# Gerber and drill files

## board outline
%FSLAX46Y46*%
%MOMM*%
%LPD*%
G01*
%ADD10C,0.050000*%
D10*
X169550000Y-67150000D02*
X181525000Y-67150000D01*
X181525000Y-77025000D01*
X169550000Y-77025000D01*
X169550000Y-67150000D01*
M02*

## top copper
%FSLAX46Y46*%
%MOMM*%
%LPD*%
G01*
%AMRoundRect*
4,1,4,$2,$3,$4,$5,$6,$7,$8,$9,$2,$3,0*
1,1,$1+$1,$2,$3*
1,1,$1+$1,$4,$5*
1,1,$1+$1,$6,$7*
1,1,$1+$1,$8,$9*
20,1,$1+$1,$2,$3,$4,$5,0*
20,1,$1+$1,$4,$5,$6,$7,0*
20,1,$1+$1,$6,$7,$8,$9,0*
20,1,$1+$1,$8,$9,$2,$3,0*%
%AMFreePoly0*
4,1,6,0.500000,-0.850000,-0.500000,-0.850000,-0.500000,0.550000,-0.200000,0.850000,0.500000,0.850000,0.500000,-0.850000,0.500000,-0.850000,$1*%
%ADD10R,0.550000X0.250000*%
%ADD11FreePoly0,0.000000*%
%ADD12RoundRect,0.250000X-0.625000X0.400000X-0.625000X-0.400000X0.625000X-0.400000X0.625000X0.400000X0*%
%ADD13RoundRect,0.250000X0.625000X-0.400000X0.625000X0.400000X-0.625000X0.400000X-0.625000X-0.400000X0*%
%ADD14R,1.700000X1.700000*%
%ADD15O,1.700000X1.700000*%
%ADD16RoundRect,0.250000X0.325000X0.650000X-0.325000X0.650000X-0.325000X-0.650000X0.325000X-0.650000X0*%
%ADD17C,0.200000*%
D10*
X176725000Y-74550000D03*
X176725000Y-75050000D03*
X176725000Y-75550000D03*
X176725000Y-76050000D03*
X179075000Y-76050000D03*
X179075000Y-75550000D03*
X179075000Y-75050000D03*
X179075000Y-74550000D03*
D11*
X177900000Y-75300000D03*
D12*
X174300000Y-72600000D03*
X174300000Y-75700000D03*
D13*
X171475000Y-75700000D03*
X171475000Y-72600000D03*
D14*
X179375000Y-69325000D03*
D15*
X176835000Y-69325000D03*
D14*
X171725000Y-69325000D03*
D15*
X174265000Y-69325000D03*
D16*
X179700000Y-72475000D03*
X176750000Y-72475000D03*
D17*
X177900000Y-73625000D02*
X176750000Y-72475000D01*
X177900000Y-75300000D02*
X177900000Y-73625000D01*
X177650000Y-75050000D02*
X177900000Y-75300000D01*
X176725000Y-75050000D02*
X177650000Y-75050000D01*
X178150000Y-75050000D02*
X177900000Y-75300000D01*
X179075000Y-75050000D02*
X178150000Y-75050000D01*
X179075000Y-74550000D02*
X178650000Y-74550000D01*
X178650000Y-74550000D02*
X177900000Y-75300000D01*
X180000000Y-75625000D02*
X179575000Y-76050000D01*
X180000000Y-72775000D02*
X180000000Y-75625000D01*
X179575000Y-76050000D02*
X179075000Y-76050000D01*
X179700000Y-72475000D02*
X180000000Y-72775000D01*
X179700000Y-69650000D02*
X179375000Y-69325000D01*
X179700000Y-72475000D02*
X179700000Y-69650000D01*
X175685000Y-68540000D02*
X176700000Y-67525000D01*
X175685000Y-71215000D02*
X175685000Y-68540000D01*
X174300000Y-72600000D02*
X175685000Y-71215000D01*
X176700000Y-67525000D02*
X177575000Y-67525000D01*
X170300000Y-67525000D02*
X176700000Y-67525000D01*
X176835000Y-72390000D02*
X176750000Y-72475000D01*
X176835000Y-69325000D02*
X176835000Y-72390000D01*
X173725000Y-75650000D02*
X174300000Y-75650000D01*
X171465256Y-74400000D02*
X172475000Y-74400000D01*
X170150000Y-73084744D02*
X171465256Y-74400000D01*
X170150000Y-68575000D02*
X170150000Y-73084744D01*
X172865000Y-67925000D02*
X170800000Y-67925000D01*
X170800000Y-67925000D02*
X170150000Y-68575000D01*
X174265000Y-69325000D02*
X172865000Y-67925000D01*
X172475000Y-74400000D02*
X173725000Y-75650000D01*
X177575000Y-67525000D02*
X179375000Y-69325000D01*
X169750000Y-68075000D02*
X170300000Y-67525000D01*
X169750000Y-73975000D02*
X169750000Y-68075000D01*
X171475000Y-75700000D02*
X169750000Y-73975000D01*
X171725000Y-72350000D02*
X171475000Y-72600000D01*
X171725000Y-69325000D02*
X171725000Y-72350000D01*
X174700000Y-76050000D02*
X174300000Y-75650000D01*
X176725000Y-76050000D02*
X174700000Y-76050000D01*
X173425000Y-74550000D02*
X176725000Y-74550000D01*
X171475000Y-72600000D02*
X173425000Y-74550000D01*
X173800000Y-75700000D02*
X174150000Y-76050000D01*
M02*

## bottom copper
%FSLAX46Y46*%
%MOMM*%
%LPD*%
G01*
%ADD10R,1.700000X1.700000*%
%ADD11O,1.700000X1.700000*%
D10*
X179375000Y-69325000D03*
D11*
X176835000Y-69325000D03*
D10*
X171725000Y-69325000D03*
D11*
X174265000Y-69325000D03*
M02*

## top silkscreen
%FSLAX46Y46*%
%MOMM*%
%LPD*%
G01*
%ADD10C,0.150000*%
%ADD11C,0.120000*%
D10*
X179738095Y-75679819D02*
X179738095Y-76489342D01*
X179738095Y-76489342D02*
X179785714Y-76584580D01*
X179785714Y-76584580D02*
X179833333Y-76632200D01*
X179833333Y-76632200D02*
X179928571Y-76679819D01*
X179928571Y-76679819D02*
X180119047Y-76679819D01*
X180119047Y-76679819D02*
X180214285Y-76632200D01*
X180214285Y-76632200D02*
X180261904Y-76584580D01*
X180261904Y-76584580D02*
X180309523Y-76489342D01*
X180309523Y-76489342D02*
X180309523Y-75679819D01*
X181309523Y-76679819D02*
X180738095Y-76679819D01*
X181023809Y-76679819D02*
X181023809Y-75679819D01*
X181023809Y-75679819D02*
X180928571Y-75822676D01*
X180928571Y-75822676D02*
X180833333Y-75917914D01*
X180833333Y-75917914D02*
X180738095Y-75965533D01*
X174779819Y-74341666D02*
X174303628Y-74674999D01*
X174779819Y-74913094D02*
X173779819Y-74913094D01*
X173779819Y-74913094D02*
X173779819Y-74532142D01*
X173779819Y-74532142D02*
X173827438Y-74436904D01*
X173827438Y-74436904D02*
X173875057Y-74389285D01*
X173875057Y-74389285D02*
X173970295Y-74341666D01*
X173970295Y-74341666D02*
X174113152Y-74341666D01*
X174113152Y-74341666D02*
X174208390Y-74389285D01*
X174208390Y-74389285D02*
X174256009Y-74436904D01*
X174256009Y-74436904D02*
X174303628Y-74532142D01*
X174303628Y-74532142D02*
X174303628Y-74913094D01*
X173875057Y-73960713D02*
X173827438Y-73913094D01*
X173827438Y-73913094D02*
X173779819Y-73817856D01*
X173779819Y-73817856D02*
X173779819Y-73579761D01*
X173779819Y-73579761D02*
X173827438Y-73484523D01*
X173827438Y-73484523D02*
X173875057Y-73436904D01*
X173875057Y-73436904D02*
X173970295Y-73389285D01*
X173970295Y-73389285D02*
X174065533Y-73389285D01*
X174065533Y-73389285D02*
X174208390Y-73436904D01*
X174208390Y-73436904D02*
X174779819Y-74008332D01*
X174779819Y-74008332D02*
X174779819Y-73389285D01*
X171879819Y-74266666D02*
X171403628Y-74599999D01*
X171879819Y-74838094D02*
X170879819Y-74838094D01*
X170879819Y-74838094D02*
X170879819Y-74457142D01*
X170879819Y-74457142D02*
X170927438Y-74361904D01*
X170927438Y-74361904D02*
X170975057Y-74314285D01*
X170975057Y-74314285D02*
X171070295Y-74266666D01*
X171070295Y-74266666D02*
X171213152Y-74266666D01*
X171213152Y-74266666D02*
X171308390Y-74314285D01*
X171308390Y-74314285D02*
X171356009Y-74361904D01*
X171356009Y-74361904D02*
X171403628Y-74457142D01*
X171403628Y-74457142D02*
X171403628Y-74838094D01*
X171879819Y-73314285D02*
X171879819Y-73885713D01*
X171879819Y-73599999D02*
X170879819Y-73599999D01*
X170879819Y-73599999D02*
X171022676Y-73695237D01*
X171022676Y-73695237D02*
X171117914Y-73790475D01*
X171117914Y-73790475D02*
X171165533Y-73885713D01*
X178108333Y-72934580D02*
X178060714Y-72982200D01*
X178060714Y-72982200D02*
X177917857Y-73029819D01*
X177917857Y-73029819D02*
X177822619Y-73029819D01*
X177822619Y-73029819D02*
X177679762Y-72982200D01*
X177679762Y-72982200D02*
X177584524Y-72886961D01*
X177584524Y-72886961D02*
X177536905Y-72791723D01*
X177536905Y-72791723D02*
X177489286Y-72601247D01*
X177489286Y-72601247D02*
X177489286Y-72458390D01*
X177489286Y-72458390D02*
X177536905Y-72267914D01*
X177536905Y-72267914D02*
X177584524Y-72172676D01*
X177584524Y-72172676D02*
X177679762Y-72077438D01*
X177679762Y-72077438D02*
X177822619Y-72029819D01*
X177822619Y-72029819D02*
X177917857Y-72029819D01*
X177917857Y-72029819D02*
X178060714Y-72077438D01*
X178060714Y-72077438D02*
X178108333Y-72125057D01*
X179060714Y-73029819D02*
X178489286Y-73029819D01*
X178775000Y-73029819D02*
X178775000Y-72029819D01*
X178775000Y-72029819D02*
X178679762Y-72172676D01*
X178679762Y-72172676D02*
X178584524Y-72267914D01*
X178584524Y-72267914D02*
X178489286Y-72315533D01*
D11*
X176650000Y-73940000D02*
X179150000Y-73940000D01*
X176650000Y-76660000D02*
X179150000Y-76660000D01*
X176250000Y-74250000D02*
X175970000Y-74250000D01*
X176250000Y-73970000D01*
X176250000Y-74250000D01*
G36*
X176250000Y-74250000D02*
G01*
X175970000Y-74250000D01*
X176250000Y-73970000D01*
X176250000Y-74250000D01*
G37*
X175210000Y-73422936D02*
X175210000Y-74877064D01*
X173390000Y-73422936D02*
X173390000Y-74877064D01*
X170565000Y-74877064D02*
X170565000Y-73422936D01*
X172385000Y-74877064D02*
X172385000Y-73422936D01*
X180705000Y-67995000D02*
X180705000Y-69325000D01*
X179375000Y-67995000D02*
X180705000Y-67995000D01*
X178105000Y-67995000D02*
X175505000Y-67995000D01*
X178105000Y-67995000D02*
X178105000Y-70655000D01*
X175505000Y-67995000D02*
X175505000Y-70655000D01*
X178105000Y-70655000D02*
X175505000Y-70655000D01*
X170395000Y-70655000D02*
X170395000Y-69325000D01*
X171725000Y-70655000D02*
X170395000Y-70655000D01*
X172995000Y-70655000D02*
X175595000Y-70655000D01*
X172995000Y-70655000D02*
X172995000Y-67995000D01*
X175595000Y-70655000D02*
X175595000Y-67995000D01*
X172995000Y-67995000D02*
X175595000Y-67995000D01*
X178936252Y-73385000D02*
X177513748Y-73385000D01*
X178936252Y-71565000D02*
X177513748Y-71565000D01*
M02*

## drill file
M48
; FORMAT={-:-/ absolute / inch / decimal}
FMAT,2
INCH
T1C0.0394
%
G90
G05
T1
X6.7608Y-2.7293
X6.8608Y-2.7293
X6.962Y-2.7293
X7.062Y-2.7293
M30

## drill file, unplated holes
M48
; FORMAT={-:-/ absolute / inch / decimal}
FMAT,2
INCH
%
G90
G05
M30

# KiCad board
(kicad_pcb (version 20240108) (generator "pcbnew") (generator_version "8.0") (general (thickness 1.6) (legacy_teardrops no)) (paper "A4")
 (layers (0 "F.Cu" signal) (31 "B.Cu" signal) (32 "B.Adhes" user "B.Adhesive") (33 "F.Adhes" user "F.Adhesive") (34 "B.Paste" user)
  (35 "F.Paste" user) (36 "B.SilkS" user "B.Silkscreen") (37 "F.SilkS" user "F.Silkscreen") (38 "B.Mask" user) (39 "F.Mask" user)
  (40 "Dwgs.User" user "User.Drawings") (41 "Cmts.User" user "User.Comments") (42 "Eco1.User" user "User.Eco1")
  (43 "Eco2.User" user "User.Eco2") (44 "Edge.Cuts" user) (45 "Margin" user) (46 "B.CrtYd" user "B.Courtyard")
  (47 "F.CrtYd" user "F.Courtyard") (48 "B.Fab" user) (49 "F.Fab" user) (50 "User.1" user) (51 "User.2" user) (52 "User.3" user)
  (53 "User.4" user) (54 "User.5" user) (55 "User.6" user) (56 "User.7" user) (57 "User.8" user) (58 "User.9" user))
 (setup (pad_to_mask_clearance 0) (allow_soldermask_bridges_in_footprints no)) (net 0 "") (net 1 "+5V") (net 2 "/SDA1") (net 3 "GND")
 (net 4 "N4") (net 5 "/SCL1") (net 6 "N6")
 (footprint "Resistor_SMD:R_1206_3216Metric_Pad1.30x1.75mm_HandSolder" (layer "F.Cu") (at 171.475 74.15 90)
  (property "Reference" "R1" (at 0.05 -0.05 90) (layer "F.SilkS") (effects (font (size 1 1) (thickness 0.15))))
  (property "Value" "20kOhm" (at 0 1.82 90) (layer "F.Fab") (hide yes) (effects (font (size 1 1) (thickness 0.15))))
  (fp_line (start -0.727064 -0.91) (end 0.727064 -0.91) (stroke (width 0.12) (type solid)) (layer "F.SilkS"))
  (fp_line (start -0.727064 0.91) (end 0.727064 0.91) (stroke (width 0.12) (type solid)) (layer "F.SilkS"))
  (pad "1" smd roundrect (at -1.55 0 90) (size 1.3 1.75) (layers "F.Cu" "F.Paste" "F.Mask") (roundrect_rratio 0.192308) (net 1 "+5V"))
  (pad "2" smd roundrect (at 1.55 0 90) (size 1.3 1.75) (layers "F.Cu" "F.Paste" "F.Mask") (roundrect_rratio 0.192308) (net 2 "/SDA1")))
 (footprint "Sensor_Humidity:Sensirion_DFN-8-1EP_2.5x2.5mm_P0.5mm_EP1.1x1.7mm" (layer "F.Cu") (at 177.9 75.3)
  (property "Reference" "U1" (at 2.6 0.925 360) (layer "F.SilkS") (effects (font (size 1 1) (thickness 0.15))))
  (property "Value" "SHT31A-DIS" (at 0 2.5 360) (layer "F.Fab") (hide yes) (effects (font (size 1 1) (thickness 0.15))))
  (fp_line (start -1.25 -1.36) (end 1.25 -1.36) (stroke (width 0.12) (type solid)) (layer "F.SilkS"))
  (fp_line (start -1.25 1.36) (end 1.25 1.36) (stroke (width 0.12) (type solid)) (layer "F.SilkS"))
  (fp_poly
   (pts (xy -1.65 -1.05) (xy -1.93 -1.05) (xy -1.65 -1.33) (xy -1.65 -1.05)) (stroke (width 0.12) (type solid)) (fill solid)
   (layer "F.SilkS"))
  (pad "" smd custom (at 0 0) (size 0.9 0.9) (layers "F.Paste") (zone_connect 0) (thermal_bridge_angle 45)
   (options (clearance outline) (anchor rect)) (primitives))
  (pad "1" smd rect (at -1.175 -0.75) (size 0.55 0.25) (layers "F.Cu" "F.Paste" "F.Mask") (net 2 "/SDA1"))
  (pad "2" smd rect (at -1.175 -0.25) (size 0.55 0.25) (layers "F.Cu" "F.Paste" "F.Mask") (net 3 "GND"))
  (pad "3" smd rect (at -1.175 0.25) (size 0.55 0.25) (layers "F.Cu" "F.Paste" "F.Mask") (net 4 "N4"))
  (pad "4" smd rect (at -1.175 0.75 180) (size 0.55 0.25) (layers "F.Cu" "F.Paste" "F.Mask") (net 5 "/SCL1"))
  (pad "5" smd rect (at 1.175 0.75) (size 0.55 0.25) (layers "F.Cu" "F.Paste" "F.Mask") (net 1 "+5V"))
  (pad "6" smd rect (at 1.175 0.25) (size 0.55 0.25) (layers "F.Cu" "F.Paste" "F.Mask") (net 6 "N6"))
  (pad "7" smd rect (at 1.175 -0.25) (size 0.55 0.25) (layers "F.Cu" "F.Paste" "F.Mask") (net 3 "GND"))
  (pad "8" smd rect (at 1.175 -0.75) (size 0.55 0.25) (layers "F.Cu" "F.Paste" "F.Mask") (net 3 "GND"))
  (pad "9" smd custom (at 0 0) (size 1 1) (layers "F.Cu" "F.Mask") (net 3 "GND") (zone_connect 0)
   (options (clearance outline) (anchor circle)) (primitives)))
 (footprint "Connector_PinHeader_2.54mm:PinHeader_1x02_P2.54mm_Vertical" (layer "F.Cu") (at 171.725 69.325 90)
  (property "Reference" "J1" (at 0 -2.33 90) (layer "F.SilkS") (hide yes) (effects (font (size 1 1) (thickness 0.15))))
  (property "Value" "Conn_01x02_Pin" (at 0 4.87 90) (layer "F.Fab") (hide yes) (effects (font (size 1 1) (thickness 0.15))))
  (fp_line (start -1.33 -1.33) (end 0 -1.33) (stroke (width 0.12) (type solid)) (layer "F.SilkS"))
  (fp_line (start -1.33 0) (end -1.33 -1.33) (stroke (width 0.12) (type solid)) (layer "F.SilkS"))
  (fp_line (start 1.33 1.27) (end 1.33 3.87) (stroke (width 0.12) (type solid)) (layer "F.SilkS"))
  (fp_line (start -1.33 1.27) (end 1.33 1.27) (stroke (width 0.12) (type solid)) (layer "F.SilkS"))
  (fp_line (start -1.33 1.27) (end -1.33 3.87) (stroke (width 0.12) (type solid)) (layer "F.SilkS"))
  (fp_line (start -1.33 3.87) (end 1.33 3.87) (stroke (width 0.12) (type solid)) (layer "F.SilkS"))
  (pad "1" thru_hole rect (at 0 0 90) (size 1.7 1.7) (drill 1) (layers "*.Cu" "*.Mask") (remove_unused_layers no) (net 2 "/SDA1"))
  (pad "2" thru_hole oval (at 0 2.54 90) (size 1.7 1.7) (drill 1) (layers "*.Cu" "*.Mask") (remove_unused_layers no) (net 5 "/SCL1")))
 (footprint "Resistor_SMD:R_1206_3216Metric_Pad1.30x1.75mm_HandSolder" (layer "F.Cu") (at 174.3 74.15 -90)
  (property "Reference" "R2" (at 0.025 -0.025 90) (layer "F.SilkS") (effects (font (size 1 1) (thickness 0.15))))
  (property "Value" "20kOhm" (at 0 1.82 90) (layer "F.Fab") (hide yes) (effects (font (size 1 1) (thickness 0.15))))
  (fp_line (start -0.727064 0.91) (end 0.727064 0.91) (stroke (width 0.12) (type solid)) (layer "F.SilkS"))
  (fp_line (start -0.727064 -0.91) (end 0.727064 -0.91) (stroke (width 0.12) (type solid)) (layer "F.SilkS"))
  (pad "1" smd roundrect (at -1.55 0 270) (size 1.3 1.75) (layers "F.Cu" "F.Paste" "F.Mask") (roundrect_rratio 0.192308) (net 1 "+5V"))
  (pad "2" smd roundrect (at 1.55 0 270) (size 1.3 1.75) (layers "F.Cu" "F.Paste" "F.Mask") (roundrect_rratio 0.192308) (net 5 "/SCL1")))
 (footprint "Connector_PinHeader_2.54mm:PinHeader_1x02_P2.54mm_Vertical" (layer "F.Cu") (at 179.375 69.325 -90)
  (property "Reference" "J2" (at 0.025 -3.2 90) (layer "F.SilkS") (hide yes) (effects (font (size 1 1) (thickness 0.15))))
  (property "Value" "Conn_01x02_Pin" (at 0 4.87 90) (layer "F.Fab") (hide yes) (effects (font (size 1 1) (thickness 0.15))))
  (fp_line (start -1.33 3.87) (end 1.33 3.87) (stroke (width 0.12) (type solid)) (layer "F.SilkS"))
  (fp_line (start -1.33 1.27) (end -1.33 3.87) (stroke (width 0.12) (type solid)) (layer "F.SilkS"))
  (fp_line (start -1.33 1.27) (end 1.33 1.27) (stroke (width 0.12) (type solid)) (layer "F.SilkS"))
  (fp_line (start 1.33 1.27) (end 1.33 3.87) (stroke (width 0.12) (type solid)) (layer "F.SilkS"))
  (fp_line (start -1.33 0) (end -1.33 -1.33) (stroke (width 0.12) (type solid)) (layer "F.SilkS"))
  (fp_line (start -1.33 -1.33) (end 0 -1.33) (stroke (width 0.12) (type solid)) (layer "F.SilkS"))
  (pad "1" thru_hole rect (at 0 0 270) (size 1.7 1.7) (drill 1) (layers "*.Cu" "*.Mask") (remove_unused_layers no) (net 1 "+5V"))
  (pad "2" thru_hole oval (at 0 2.54 270) (size 1.7 1.7) (drill 1) (layers "*.Cu" "*.Mask") (remove_unused_layers no) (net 3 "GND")))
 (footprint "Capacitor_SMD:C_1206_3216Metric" (layer "F.Cu") (at 178.225 72.475 180)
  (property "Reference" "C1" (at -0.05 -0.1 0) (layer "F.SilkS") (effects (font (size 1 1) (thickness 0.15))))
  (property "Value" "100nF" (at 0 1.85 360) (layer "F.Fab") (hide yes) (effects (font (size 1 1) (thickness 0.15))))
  (fp_line (start -0.711252 0.91) (end 0.711252 0.91) (stroke (width 0.12) (type solid)) (layer "F.SilkS"))
  (fp_line (start -0.711252 -0.91) (end 0.711252 -0.91) (stroke (width 0.12) (type solid)) (layer "F.SilkS"))
  (pad "1" smd roundrect (at -1.475 0 180) (size 1.15 1.8) (layers "F.Cu" "F.Paste" "F.Mask") (roundrect_rratio 0.217391) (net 1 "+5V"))
  (pad "2" smd roundrect (at 1.475 0 180) (size 1.15 1.8) (layers "F.Cu" "F.Paste" "F.Mask") (roundrect_rratio 0.217391) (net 3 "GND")))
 (gr_rect (start 169.55 67.15) (end 181.525 77.025) (stroke (width 0.05) (type default)) (fill none) (layer "Edge.Cuts"))
 (segment (start 176.7 67.525) (end 177.575 67.525) (width 0.2) (layer "F.Cu") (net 1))
 (segment (start 179.7 72.475) (end 180 72.775) (width 0.2) (layer "F.Cu") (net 1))
 (segment (start 169.75 73.975) (end 169.75 68.075) (width 0.2) (layer "F.Cu") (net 1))
 (segment (start 179.7 69.65) (end 179.375 69.325) (width 0.2) (layer "F.Cu") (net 1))
 (segment (start 180 72.775) (end 180 75.625) (width 0.2) (layer "F.Cu") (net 1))
 (segment (start 177.575 67.525) (end 179.375 69.325) (width 0.2) (layer "F.Cu") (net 1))
 (segment (start 180 75.625) (end 179.575 76.05) (width 0.2) (layer "F.Cu") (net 1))
 (segment (start 169.75 68.075) (end 170.3 67.525) (width 0.2) (layer "F.Cu") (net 1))
 (segment (start 179.575 76.05) (end 179.075 76.05) (width 0.2) (layer "F.Cu") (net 1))
 (segment (start 179.7 72.475) (end 179.7 69.65) (width 0.2) (layer "F.Cu") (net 1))
 (segment (start 170.3 67.525) (end 176.7 67.525) (width 0.2) (layer "F.Cu") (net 1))
 (segment (start 171.475 75.7) (end 169.75 73.975) (width 0.2) (layer "F.Cu") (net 1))
 (segment (start 175.685 71.215) (end 175.685 68.54) (width 0.2) (layer "F.Cu") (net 1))
 (segment (start 175.685 68.54) (end 176.7 67.525) (width 0.2) (layer "F.Cu") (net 1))
 (segment (start 174.3 72.6) (end 175.685 71.215) (width 0.2) (layer "F.Cu") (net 1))
 (segment (start 178.15 75.05) (end 177.9 75.3) (width 0.2) (layer "F.Cu") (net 3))
 (segment (start 176.835 72.39) (end 176.75 72.475) (width 0.2) (layer "F.Cu") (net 3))
 (segment (start 179.075 74.55) (end 178.65 74.55) (width 0.2) (layer "F.Cu") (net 3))
 (segment (start 176.835 69.325) (end 176.835 72.39) (width 0.2) (layer "F.Cu") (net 3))
 (segment (start 176.725 75.05) (end 177.65 75.05) (width 0.2) (layer "F.Cu") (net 3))
 (segment (start 177.65 75.05) (end 177.9 75.3) (width 0.2) (layer "F.Cu") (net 3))
 (segment (start 179.075 75.05) (end 178.15 75.05) (width 0.2) (layer "F.Cu") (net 3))
 (segment (start 177.9 75.3) (end 177.9 73.625) (width 0.2) (layer "F.Cu") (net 3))
 (segment (start 178.65 74.55) (end 177.9 75.3) (width 0.2) (layer "F.Cu") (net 3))
 (segment (start 177.9 73.625) (end 176.75 72.475) (width 0.2) (layer "F.Cu") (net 3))
 (segment (start 174.265 69.325) (end 172.865 67.925) (width 0.2) (layer "F.Cu") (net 5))
 (segment (start 170.8 67.925) (end 170.15 68.575) (width 0.2) (layer "F.Cu") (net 5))
 (segment (start 176.725 76.05) (end 174.7 76.05) (width 0.2) (layer "F.Cu") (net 5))
 (segment (start 170.15 68.575) (end 170.15 73.084744) (width 0.2) (layer "F.Cu") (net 5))
 (segment (start 170.15 73.084744) (end 171.465256 74.4) (width 0.2) (layer "F.Cu") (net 5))
 (segment (start 172.475 74.4) (end 173.725 75.65) (width 0.2) (layer "F.Cu") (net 5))
 (segment (start 171.465256 74.4) (end 172.475 74.4) (width 0.2) (layer "F.Cu") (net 5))
 (segment (start 173.8 75.7) (end 174.15 76.05) (width 0.2) (layer "F.Cu") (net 5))
 (segment (start 172.865 67.925) (end 170.8 67.925) (width 0.2) (layer "F.Cu") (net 5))
 (segment (start 173.725 75.65) (end 174.3 75.65) (width 0.2) (layer "F.Cu") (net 5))
 (segment (start 174.7 76.05) (end 174.3 75.65) (width 0.2) (layer "F.Cu") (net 5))
 (segment (start 171.725 69.325) (end 171.725 72.35) (width 0.2) (layer "F.Cu") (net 2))
 (segment (start 171.725 72.35) (end 171.475 72.6) (width 0.2) (layer "F.Cu") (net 2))
 (segment (start 171.475 72.6) (end 173.425 74.55) (width 0.2) (layer "F.Cu") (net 2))
 (segment (start 173.425 74.55) (end 176.725 74.55) (width 0.2) (layer "F.Cu") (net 2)))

